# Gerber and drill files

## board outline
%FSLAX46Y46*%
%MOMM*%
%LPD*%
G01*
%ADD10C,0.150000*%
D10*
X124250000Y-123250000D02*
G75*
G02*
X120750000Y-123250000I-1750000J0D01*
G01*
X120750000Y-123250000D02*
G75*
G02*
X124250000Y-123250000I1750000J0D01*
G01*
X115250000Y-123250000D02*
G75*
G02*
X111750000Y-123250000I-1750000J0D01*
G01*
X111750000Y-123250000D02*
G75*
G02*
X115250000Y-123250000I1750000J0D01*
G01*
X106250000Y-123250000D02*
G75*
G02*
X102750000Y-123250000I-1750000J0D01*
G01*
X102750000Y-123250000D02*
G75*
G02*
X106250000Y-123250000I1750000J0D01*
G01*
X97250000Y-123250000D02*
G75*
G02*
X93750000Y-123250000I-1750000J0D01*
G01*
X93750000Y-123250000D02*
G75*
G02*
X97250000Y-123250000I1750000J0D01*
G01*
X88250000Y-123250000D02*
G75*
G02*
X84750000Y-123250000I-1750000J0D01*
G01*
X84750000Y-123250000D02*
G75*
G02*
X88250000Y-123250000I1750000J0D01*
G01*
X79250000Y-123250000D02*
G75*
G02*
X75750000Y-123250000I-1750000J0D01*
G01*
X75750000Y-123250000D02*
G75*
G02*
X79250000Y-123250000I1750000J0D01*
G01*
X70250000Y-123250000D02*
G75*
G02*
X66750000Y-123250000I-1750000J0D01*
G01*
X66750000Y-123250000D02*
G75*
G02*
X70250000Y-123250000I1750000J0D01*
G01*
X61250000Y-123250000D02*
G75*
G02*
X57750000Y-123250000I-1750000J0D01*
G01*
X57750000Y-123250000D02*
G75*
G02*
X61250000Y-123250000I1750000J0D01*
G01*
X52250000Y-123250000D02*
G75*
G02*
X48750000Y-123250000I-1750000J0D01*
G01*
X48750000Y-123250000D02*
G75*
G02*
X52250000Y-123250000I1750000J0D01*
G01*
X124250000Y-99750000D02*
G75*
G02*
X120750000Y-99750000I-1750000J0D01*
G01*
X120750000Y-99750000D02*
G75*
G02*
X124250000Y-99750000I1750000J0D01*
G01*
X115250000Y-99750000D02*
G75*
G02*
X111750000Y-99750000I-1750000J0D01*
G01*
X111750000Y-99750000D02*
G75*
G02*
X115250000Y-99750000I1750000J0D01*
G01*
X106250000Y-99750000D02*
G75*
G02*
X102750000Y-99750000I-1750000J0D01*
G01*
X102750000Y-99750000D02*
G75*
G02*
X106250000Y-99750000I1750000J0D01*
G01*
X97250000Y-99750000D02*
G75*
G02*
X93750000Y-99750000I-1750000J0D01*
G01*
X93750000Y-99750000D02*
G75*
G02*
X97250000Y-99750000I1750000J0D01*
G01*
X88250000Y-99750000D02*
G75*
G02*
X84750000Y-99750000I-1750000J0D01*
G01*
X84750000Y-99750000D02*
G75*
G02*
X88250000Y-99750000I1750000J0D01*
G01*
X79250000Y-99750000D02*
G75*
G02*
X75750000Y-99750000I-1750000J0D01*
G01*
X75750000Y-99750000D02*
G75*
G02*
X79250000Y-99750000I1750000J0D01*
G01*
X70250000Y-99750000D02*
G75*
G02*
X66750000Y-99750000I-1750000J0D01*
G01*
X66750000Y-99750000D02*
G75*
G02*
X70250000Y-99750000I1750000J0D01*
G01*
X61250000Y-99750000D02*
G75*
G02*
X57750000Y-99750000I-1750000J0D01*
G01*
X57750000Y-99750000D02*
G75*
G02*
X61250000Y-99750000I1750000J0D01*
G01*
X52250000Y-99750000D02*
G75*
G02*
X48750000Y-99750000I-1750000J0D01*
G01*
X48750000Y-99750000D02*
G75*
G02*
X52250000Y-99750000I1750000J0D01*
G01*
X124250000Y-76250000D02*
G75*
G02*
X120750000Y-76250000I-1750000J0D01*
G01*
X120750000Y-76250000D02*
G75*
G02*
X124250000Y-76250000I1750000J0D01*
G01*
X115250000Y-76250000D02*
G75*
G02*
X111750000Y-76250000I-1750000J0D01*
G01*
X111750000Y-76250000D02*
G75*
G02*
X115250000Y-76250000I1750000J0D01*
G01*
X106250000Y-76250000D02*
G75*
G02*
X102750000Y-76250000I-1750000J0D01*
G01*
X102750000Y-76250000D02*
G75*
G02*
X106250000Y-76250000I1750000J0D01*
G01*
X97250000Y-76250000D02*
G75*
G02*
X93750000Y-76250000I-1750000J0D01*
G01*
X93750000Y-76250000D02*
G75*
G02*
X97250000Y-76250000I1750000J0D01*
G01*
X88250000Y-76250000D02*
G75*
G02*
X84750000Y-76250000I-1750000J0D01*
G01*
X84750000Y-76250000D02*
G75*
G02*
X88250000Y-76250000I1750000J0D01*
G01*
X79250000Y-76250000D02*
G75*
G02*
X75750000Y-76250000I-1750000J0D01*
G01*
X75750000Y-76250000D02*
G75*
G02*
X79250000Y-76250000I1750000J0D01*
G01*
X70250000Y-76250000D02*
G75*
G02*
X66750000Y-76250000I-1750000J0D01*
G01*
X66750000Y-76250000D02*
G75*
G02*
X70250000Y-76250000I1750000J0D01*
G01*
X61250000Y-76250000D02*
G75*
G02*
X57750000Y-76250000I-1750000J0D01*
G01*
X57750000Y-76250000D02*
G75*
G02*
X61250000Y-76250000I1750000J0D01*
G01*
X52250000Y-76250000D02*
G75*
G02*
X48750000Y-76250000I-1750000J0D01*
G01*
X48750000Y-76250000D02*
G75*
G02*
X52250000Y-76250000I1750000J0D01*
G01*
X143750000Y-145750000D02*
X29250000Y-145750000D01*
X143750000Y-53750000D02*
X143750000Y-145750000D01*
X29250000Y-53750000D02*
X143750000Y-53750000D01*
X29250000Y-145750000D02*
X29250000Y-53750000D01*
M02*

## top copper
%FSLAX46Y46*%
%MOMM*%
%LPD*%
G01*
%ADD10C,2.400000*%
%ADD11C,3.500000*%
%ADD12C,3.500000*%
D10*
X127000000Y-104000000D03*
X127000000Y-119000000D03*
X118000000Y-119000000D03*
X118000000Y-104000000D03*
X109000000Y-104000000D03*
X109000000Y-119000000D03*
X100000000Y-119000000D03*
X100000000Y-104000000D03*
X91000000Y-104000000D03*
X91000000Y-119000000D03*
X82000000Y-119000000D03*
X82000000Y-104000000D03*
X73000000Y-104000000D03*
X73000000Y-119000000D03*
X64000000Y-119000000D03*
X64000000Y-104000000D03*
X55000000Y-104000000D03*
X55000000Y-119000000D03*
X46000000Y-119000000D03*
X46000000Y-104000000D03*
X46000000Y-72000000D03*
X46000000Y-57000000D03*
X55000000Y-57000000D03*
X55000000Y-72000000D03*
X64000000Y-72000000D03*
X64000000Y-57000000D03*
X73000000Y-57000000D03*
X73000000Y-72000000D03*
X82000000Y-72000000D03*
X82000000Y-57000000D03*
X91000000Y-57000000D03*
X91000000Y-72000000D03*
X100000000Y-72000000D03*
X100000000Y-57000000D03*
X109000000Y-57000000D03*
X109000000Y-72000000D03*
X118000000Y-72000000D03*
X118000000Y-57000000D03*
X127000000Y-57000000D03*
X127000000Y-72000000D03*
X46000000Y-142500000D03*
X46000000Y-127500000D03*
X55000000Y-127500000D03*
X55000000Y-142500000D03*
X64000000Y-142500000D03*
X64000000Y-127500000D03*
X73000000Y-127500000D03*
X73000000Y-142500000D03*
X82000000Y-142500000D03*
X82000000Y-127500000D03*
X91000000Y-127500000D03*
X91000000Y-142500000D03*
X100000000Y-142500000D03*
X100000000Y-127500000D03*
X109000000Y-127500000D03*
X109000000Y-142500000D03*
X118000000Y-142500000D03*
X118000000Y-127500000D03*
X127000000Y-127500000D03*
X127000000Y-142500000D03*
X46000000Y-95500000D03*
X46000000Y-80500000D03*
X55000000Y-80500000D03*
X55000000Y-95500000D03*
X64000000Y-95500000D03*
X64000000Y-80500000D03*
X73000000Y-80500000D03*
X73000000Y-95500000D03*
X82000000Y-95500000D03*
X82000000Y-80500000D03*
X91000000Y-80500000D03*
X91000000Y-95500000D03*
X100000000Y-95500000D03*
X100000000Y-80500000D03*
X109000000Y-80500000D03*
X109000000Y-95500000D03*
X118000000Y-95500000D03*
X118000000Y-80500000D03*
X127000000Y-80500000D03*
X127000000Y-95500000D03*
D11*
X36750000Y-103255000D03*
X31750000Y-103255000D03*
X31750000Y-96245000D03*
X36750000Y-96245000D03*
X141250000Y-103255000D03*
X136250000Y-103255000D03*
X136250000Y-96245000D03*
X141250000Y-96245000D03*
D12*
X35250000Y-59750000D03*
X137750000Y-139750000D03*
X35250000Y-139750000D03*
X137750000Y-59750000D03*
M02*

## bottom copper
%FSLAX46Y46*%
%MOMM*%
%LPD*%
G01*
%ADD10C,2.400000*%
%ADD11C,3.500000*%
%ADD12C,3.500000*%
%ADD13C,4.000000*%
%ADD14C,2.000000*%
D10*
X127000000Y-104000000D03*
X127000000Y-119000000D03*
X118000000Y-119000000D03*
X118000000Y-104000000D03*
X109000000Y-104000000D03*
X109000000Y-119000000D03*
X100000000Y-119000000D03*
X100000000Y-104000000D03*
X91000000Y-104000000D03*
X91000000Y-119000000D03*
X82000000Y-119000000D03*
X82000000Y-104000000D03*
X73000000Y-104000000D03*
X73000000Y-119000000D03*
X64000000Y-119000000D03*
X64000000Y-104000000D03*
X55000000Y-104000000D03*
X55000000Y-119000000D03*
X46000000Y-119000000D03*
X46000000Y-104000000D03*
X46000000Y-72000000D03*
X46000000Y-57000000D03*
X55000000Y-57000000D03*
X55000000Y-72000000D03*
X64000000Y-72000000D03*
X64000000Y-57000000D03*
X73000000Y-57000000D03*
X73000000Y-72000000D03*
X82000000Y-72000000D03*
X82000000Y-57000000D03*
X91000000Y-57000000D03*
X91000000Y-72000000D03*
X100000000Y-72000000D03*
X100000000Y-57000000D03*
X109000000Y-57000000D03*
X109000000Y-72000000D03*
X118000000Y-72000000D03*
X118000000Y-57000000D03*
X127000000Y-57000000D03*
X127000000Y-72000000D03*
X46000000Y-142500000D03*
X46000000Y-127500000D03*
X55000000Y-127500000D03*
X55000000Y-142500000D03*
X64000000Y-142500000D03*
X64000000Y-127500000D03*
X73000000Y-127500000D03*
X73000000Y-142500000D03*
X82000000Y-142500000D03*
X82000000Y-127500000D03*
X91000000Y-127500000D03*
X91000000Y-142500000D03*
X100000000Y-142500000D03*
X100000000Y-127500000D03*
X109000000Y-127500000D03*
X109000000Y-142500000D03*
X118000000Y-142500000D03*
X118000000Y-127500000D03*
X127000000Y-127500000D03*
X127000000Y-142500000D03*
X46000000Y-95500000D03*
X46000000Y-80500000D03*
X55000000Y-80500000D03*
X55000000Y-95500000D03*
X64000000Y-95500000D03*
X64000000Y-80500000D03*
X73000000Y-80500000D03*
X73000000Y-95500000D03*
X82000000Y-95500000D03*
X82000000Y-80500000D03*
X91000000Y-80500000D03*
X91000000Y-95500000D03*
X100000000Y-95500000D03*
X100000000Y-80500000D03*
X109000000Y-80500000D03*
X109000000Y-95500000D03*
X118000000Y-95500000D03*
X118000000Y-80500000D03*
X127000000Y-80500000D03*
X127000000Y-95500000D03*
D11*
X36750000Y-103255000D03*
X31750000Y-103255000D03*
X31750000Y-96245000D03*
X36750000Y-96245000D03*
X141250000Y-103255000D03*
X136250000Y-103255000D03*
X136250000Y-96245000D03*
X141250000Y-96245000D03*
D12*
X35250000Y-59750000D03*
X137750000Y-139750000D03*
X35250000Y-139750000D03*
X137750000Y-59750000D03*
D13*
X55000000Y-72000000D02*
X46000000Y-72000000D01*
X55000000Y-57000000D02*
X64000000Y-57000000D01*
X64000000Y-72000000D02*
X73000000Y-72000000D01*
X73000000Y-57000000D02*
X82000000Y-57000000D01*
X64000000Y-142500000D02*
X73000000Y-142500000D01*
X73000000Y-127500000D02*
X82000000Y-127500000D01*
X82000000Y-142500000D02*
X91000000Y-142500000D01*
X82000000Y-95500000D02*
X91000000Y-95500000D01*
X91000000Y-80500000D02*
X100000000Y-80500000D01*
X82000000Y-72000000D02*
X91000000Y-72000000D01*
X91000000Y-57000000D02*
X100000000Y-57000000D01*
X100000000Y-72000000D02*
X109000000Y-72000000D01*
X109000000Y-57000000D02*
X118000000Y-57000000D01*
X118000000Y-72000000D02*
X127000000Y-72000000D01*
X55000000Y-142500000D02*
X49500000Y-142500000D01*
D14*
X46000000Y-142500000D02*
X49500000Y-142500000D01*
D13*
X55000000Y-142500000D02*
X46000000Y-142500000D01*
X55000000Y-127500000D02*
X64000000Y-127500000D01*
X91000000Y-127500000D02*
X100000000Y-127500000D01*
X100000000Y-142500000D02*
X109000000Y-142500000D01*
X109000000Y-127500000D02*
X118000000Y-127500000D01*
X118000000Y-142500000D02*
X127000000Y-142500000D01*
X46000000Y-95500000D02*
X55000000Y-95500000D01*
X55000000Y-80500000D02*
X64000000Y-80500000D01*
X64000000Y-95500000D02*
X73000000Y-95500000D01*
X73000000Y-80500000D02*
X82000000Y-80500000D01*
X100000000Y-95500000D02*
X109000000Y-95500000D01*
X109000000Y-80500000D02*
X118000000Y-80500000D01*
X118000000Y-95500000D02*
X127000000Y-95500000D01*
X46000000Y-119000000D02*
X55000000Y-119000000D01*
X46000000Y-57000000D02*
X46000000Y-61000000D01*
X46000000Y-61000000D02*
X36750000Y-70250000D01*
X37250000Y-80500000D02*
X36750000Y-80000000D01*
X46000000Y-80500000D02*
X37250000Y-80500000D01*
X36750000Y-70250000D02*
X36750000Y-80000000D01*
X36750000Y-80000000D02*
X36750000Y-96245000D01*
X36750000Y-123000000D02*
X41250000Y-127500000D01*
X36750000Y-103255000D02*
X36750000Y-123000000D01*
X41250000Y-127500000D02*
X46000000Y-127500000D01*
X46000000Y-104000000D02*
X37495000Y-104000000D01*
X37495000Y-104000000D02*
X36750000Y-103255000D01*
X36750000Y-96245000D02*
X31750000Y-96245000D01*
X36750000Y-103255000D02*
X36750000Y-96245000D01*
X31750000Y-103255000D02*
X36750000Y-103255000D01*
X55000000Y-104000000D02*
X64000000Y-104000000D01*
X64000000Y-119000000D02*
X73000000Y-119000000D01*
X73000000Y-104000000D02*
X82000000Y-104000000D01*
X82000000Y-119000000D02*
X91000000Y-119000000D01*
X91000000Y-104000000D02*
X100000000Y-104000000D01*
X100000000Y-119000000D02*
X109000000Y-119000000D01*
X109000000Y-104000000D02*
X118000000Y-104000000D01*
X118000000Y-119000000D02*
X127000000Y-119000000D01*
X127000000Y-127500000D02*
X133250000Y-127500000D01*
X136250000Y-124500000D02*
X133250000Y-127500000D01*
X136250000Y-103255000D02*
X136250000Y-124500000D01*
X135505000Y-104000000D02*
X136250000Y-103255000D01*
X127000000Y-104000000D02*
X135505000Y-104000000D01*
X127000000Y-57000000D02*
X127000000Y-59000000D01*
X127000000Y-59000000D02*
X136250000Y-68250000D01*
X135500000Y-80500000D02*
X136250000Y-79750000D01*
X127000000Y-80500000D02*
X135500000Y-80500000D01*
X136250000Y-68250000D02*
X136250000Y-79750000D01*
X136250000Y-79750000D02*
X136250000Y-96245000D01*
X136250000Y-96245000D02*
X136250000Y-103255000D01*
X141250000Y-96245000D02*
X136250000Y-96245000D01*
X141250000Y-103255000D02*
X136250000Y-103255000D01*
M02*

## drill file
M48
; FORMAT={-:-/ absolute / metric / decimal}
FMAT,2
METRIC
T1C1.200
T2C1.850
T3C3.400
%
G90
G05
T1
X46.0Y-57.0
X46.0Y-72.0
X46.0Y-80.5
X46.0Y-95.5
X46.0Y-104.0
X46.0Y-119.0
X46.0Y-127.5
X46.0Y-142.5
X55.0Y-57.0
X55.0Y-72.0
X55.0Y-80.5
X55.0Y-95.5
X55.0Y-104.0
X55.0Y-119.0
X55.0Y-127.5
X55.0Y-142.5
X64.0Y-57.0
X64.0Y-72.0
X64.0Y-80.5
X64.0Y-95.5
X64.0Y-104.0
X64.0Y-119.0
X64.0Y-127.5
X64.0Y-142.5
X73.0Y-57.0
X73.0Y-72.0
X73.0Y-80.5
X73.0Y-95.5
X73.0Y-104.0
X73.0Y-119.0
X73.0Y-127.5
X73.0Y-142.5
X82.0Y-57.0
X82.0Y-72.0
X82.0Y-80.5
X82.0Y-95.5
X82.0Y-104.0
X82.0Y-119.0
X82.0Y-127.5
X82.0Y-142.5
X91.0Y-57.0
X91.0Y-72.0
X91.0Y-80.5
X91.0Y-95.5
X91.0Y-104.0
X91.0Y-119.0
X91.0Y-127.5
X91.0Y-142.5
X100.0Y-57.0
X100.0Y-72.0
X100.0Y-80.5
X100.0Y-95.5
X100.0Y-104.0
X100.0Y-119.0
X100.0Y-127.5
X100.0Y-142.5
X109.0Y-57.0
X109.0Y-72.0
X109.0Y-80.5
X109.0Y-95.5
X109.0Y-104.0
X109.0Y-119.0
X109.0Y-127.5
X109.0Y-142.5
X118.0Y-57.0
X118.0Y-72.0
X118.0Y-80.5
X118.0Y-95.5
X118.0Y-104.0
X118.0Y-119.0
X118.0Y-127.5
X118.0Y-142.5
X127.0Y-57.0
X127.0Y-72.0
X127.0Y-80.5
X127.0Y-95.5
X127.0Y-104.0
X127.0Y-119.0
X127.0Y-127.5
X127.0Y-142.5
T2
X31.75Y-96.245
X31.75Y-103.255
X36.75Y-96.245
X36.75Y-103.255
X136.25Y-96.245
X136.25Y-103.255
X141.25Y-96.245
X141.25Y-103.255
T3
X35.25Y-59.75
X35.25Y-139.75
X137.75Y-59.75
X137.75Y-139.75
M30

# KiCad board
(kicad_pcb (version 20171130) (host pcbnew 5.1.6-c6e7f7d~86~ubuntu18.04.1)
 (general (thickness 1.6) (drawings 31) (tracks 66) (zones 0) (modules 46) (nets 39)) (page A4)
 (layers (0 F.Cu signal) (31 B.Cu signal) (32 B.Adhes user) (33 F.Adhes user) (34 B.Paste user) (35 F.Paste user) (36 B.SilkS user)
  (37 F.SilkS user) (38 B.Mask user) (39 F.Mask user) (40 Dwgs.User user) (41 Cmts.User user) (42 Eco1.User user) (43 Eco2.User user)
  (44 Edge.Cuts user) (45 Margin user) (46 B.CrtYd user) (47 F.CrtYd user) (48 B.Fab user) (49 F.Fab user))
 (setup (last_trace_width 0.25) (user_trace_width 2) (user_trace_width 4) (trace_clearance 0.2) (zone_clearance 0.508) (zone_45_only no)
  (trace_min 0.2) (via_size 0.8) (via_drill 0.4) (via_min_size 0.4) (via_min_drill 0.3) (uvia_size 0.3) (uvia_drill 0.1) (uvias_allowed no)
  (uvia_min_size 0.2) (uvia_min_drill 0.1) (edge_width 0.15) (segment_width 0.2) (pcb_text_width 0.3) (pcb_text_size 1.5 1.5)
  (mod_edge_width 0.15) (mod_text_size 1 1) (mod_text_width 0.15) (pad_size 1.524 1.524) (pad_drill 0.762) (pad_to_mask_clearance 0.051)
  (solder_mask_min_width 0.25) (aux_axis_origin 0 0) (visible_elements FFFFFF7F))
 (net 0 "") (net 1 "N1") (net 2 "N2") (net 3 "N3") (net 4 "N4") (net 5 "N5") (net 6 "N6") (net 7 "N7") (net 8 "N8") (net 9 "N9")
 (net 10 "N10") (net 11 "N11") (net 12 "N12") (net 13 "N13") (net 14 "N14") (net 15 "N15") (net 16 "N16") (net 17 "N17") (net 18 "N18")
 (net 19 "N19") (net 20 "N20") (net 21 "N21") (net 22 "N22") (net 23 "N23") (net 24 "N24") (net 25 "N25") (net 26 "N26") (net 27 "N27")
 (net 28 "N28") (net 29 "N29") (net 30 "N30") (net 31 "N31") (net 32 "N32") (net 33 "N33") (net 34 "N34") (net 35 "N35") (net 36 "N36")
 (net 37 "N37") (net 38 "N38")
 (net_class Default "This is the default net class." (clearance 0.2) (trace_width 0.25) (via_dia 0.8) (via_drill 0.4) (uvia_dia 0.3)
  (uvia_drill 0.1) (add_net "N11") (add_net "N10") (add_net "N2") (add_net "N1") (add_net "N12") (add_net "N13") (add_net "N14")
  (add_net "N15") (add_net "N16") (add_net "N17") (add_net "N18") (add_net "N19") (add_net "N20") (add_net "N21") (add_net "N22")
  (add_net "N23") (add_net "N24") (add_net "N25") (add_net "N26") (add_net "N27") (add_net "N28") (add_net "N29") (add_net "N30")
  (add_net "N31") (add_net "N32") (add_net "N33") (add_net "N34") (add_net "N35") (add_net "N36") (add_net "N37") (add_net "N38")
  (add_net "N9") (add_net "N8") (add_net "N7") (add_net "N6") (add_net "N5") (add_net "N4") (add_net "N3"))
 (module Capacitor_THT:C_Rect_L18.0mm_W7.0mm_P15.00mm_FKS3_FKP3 (layer F.Cu) (at 127 119 90)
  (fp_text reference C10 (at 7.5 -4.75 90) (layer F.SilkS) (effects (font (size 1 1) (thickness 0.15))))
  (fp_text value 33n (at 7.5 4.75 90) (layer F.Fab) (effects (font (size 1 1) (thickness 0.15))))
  (pad 2 thru_hole circle (at 15 0 90) (size 2.4 2.4) (drill 1.2) (layers *.Cu *.Mask) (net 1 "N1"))
  (pad 1 thru_hole circle (at 0 0 90) (size 2.4 2.4) (drill 1.2) (layers *.Cu *.Mask) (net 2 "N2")))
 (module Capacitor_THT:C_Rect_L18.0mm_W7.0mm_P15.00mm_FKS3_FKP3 (layer F.Cu) (at 118 104 270)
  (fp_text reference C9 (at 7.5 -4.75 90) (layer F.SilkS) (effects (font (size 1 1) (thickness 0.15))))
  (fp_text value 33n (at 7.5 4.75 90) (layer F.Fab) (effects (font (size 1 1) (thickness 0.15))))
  (pad 2 thru_hole circle (at 15 0 270) (size 2.4 2.4) (drill 1.2) (layers *.Cu *.Mask) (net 2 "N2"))
  (pad 1 thru_hole circle (at 0 0 270) (size 2.4 2.4) (drill 1.2) (layers *.Cu *.Mask) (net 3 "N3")))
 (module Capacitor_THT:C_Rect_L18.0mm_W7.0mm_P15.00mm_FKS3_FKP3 (layer F.Cu) (at 109 119 90)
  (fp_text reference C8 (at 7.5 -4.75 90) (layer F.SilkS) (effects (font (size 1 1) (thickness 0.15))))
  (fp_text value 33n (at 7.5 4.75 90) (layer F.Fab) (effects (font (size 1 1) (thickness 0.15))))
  (pad 2 thru_hole circle (at 15 0 90) (size 2.4 2.4) (drill 1.2) (layers *.Cu *.Mask) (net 3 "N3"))
  (pad 1 thru_hole circle (at 0 0 90) (size 2.4 2.4) (drill 1.2) (layers *.Cu *.Mask) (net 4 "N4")))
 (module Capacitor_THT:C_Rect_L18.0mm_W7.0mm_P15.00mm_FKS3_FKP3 (layer F.Cu) (at 100 104 270)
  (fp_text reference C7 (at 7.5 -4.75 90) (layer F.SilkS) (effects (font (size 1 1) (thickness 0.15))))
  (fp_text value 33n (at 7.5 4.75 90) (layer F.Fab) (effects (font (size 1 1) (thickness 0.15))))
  (pad 2 thru_hole circle (at 15 0 270) (size 2.4 2.4) (drill 1.2) (layers *.Cu *.Mask) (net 4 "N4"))
  (pad 1 thru_hole circle (at 0 0 270) (size 2.4 2.4) (drill 1.2) (layers *.Cu *.Mask) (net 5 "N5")))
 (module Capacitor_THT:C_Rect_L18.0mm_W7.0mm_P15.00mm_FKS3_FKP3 (layer F.Cu) (at 91 119 90)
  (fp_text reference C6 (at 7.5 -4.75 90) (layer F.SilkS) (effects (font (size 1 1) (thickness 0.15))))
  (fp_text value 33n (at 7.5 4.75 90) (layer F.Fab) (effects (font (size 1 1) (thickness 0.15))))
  (pad 2 thru_hole circle (at 15 0 90) (size 2.4 2.4) (drill 1.2) (layers *.Cu *.Mask) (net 5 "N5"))
  (pad 1 thru_hole circle (at 0 0 90) (size 2.4 2.4) (drill 1.2) (layers *.Cu *.Mask) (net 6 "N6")))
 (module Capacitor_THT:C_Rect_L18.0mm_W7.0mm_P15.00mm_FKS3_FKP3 (layer F.Cu) (at 82 104 270)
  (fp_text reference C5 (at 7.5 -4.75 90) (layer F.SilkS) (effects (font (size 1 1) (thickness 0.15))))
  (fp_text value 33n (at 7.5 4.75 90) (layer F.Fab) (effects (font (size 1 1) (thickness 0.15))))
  (pad 2 thru_hole circle (at 15 0 270) (size 2.4 2.4) (drill 1.2) (layers *.Cu *.Mask) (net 6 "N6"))
  (pad 1 thru_hole circle (at 0 0 270) (size 2.4 2.4) (drill 1.2) (layers *.Cu *.Mask) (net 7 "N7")))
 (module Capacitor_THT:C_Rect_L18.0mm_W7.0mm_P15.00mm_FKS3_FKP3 (layer F.Cu) (at 73 119 90)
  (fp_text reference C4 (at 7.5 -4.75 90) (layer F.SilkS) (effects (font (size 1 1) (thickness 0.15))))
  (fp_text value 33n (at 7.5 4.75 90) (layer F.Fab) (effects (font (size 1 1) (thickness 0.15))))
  (pad 2 thru_hole circle (at 15 0 90) (size 2.4 2.4) (drill 1.2) (layers *.Cu *.Mask) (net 7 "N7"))
  (pad 1 thru_hole circle (at 0 0 90) (size 2.4 2.4) (drill 1.2) (layers *.Cu *.Mask) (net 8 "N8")))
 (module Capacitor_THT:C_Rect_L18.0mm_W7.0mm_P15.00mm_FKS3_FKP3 (layer F.Cu) (at 64 104 270)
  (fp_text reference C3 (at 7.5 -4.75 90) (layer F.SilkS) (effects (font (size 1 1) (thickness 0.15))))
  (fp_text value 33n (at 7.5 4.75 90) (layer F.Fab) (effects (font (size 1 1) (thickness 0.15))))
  (pad 2 thru_hole circle (at 15 0 270) (size 2.4 2.4) (drill 1.2) (layers *.Cu *.Mask) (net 8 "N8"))
  (pad 1 thru_hole circle (at 0 0 270) (size 2.4 2.4) (drill 1.2) (layers *.Cu *.Mask) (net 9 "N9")))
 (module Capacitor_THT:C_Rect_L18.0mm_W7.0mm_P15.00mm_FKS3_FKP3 (layer F.Cu) (at 55 119 90)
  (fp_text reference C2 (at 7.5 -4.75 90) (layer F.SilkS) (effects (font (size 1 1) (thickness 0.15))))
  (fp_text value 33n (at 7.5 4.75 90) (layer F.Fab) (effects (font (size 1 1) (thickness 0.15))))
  (pad 2 thru_hole circle (at 15 0 90) (size 2.4 2.4) (drill 1.2) (layers *.Cu *.Mask) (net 9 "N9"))
  (pad 1 thru_hole circle (at 0 0 90) (size 2.4 2.4) (drill 1.2) (layers *.Cu *.Mask) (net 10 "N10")))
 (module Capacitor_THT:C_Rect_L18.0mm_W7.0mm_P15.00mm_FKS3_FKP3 (layer F.Cu) (at 46 104 270)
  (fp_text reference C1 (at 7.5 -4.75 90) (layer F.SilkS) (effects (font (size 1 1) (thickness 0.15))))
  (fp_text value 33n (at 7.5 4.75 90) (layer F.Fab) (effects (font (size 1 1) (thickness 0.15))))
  (pad 2 thru_hole circle (at 15 0 270) (size 2.4 2.4) (drill 1.2) (layers *.Cu *.Mask) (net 10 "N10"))
  (pad 1 thru_hole circle (at 0 0 270) (size 2.4 2.4) (drill 1.2) (layers *.Cu *.Mask) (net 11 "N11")))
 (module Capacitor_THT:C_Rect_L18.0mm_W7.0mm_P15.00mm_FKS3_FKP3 (layer F.Cu) (at 46 57 270)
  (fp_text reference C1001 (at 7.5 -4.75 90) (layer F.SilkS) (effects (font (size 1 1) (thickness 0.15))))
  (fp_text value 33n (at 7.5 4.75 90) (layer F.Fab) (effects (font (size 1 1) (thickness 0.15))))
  (pad 2 thru_hole circle (at 15 0 270) (size 2.4 2.4) (drill 1.2) (layers *.Cu *.Mask) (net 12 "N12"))
  (pad 1 thru_hole circle (at 0 0 270) (size 2.4 2.4) (drill 1.2) (layers *.Cu *.Mask) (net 11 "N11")))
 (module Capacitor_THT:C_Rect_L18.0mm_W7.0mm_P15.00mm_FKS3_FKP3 (layer F.Cu) (at 55 72 90)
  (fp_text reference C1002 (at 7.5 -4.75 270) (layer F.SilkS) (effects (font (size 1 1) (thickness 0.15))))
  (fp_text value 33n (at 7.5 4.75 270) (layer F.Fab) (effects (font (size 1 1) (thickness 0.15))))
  (pad 2 thru_hole circle (at 15 0 90) (size 2.4 2.4) (drill 1.2) (layers *.Cu *.Mask) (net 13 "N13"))
  (pad 1 thru_hole circle (at 0 0 90) (size 2.4 2.4) (drill 1.2) (layers *.Cu *.Mask) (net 12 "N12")))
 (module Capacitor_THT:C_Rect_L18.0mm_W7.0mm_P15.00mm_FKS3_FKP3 (layer F.Cu) (at 64 57 270)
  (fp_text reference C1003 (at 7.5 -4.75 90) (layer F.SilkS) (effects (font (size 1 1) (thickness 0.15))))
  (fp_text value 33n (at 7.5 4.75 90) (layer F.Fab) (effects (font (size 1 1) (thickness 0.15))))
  (pad 2 thru_hole circle (at 15 0 270) (size 2.4 2.4) (drill 1.2) (layers *.Cu *.Mask) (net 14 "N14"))
  (pad 1 thru_hole circle (at 0 0 270) (size 2.4 2.4) (drill 1.2) (layers *.Cu *.Mask) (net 13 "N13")))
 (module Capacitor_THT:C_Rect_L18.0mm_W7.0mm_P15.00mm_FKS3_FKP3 (layer F.Cu) (at 73 72 90)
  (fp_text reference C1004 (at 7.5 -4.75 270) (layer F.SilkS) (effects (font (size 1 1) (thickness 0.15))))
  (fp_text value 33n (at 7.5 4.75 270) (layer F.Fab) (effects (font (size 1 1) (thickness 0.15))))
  (pad 2 thru_hole circle (at 15 0 90) (size 2.4 2.4) (drill 1.2) (layers *.Cu *.Mask) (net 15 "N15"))
  (pad 1 thru_hole circle (at 0 0 90) (size 2.4 2.4) (drill 1.2) (layers *.Cu *.Mask) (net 14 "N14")))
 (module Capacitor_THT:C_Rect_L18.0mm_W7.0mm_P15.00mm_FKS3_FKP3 (layer F.Cu) (at 82 57 270)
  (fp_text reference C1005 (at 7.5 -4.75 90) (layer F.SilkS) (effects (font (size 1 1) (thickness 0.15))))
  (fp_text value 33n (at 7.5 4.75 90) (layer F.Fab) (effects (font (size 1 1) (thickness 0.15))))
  (pad 2 thru_hole circle (at 15 0 270) (size 2.4 2.4) (drill 1.2) (layers *.Cu *.Mask) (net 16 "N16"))
  (pad 1 thru_hole circle (at 0 0 270) (size 2.4 2.4) (drill 1.2) (layers *.Cu *.Mask) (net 15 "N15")))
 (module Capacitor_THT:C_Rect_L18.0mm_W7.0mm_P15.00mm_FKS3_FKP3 (layer F.Cu) (at 91 72 90)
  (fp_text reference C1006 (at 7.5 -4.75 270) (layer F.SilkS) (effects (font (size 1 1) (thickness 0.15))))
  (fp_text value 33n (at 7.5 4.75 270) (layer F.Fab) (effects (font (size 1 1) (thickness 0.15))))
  (pad 2 thru_hole circle (at 15 0 90) (size 2.4 2.4) (drill 1.2) (layers *.Cu *.Mask) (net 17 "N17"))
  (pad 1 thru_hole circle (at 0 0 90) (size 2.4 2.4) (drill 1.2) (layers *.Cu *.Mask) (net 16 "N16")))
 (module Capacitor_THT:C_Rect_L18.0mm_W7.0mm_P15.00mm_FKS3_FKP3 (layer F.Cu) (at 100 57 270)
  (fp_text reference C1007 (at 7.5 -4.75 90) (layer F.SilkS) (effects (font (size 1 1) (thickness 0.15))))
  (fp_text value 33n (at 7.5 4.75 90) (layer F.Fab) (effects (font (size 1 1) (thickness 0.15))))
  (pad 2 thru_hole circle (at 15 0 270) (size 2.4 2.4) (drill 1.2) (layers *.Cu *.Mask) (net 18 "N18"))
  (pad 1 thru_hole circle (at 0 0 270) (size 2.4 2.4) (drill 1.2) (layers *.Cu *.Mask) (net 17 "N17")))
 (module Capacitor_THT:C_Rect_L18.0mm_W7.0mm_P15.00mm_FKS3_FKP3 (layer F.Cu) (at 109 72 90)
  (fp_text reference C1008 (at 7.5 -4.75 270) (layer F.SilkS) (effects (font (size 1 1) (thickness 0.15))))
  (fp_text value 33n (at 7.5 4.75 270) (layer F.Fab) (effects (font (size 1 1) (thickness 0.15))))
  (pad 2 thru_hole circle (at 15 0 90) (size 2.4 2.4) (drill 1.2) (layers *.Cu *.Mask) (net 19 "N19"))
  (pad 1 thru_hole circle (at 0 0 90) (size 2.4 2.4) (drill 1.2) (layers *.Cu *.Mask) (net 18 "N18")))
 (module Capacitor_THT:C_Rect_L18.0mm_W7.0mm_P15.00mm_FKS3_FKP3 (layer F.Cu) (at 118 57 270)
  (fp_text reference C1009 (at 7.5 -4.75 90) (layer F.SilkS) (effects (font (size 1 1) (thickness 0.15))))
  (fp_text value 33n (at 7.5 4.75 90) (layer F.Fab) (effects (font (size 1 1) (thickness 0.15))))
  (pad 2 thru_hole circle (at 15 0 270) (size 2.4 2.4) (drill 1.2) (layers *.Cu *.Mask) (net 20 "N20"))
  (pad 1 thru_hole circle (at 0 0 270) (size 2.4 2.4) (drill 1.2) (layers *.Cu *.Mask) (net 19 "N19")))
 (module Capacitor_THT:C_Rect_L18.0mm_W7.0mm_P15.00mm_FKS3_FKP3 (layer F.Cu) (at 127 72 90)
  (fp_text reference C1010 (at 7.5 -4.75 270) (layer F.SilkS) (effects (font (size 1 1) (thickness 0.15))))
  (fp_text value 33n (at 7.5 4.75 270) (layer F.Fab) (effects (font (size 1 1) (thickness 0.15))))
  (pad 2 thru_hole circle (at 15 0 90) (size 2.4 2.4) (drill 1.2) (layers *.Cu *.Mask) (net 1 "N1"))
  (pad 1 thru_hole circle (at 0 0 90) (size 2.4 2.4) (drill 1.2) (layers *.Cu *.Mask) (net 20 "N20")))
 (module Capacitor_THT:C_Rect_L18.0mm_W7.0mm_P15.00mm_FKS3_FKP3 (layer F.Cu) (at 46 127.5 270)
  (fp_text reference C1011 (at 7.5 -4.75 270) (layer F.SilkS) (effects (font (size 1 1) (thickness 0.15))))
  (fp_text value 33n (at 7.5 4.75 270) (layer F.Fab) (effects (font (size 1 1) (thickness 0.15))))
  (pad 2 thru_hole circle (at 15 0 270) (size 2.4 2.4) (drill 1.2) (layers *.Cu *.Mask) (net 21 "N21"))
  (pad 1 thru_hole circle (at 0 0 270) (size 2.4 2.4) (drill 1.2) (layers *.Cu *.Mask) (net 11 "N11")))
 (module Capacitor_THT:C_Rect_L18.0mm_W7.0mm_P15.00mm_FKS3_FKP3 (layer F.Cu) (at 55 142.5 90)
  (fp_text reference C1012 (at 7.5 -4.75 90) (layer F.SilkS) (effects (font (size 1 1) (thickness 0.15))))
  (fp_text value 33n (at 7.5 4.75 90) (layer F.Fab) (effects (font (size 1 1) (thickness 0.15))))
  (pad 2 thru_hole circle (at 15 0 90) (size 2.4 2.4) (drill 1.2) (layers *.Cu *.Mask) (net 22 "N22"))
  (pad 1 thru_hole circle (at 0 0 90) (size 2.4 2.4) (drill 1.2) (layers *.Cu *.Mask) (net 21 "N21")))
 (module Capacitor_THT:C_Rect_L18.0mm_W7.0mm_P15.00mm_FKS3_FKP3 (layer F.Cu) (at 64 127.5 270)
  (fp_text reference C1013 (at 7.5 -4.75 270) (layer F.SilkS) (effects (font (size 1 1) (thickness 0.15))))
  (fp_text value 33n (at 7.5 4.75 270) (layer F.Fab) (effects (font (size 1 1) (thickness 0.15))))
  (pad 2 thru_hole circle (at 15 0 270) (size 2.4 2.4) (drill 1.2) (layers *.Cu *.Mask) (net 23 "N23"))
  (pad 1 thru_hole circle (at 0 0 270) (size 2.4 2.4) (drill 1.2) (layers *.Cu *.Mask) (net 22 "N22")))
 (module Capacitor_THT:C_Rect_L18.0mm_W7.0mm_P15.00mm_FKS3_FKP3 (layer F.Cu) (at 73 142.5 90)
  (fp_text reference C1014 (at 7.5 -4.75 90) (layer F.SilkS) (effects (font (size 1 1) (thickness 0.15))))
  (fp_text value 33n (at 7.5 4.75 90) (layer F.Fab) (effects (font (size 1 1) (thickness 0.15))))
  (pad 2 thru_hole circle (at 15 0 90) (size 2.4 2.4) (drill 1.2) (layers *.Cu *.Mask) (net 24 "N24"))
  (pad 1 thru_hole circle (at 0 0 90) (size 2.4 2.4) (drill 1.2) (layers *.Cu *.Mask) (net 23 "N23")))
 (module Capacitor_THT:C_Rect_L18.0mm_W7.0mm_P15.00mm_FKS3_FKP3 (layer F.Cu) (at 82 127.5 270)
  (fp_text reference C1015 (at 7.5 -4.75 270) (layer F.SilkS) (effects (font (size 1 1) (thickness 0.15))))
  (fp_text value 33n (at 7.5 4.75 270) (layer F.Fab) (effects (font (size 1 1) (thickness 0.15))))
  (pad 2 thru_hole circle (at 15 0 270) (size 2.4 2.4) (drill 1.2) (layers *.Cu *.Mask) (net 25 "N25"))
  (pad 1 thru_hole circle (at 0 0 270) (size 2.4 2.4) (drill 1.2) (layers *.Cu *.Mask) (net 24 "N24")))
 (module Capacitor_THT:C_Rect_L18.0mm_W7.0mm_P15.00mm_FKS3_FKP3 (layer F.Cu) (at 91 142.5 90)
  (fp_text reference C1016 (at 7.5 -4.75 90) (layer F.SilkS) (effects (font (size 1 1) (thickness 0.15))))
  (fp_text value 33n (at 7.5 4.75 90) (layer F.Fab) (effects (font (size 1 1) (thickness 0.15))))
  (pad 2 thru_hole circle (at 15 0 90) (size 2.4 2.4) (drill 1.2) (layers *.Cu *.Mask) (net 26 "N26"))
  (pad 1 thru_hole circle (at 0 0 90) (size 2.4 2.4) (drill 1.2) (layers *.Cu *.Mask) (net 25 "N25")))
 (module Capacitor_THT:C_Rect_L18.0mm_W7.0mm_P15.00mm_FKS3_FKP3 (layer F.Cu) (at 100 127.5 270)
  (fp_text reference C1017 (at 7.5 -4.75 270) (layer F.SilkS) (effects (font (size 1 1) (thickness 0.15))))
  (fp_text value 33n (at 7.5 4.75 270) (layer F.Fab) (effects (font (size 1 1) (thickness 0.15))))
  (pad 2 thru_hole circle (at 15 0 270) (size 2.4 2.4) (drill 1.2) (layers *.Cu *.Mask) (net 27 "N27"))
  (pad 1 thru_hole circle (at 0 0 270) (size 2.4 2.4) (drill 1.2) (layers *.Cu *.Mask) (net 26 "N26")))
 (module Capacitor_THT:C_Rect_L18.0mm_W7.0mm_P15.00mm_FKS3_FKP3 (layer F.Cu) (at 109 142.5 90)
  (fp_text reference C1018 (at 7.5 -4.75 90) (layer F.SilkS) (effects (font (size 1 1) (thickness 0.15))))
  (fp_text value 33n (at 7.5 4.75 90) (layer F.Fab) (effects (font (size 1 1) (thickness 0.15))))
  (pad 2 thru_hole circle (at 15 0 90) (size 2.4 2.4) (drill 1.2) (layers *.Cu *.Mask) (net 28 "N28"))
  (pad 1 thru_hole circle (at 0 0 90) (size 2.4 2.4) (drill 1.2) (layers *.Cu *.Mask) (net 27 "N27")))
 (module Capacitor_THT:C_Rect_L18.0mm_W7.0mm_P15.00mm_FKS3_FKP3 (layer F.Cu) (at 118 127.5 270)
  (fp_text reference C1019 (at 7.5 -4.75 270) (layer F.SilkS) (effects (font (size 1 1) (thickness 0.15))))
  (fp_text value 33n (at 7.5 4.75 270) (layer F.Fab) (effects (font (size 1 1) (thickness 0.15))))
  (pad 2 thru_hole circle (at 15 0 270) (size 2.4 2.4) (drill 1.2) (layers *.Cu *.Mask) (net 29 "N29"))
  (pad 1 thru_hole circle (at 0 0 270) (size 2.4 2.4) (drill 1.2) (layers *.Cu *.Mask) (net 28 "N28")))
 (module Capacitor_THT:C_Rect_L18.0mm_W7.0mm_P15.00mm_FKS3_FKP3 (layer F.Cu) (at 127 142.5 90)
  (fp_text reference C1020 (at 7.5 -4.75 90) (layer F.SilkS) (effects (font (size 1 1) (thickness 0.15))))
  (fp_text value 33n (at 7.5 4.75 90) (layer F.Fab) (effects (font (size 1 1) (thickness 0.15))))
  (pad 2 thru_hole circle (at 15 0 90) (size 2.4 2.4) (drill 1.2) (layers *.Cu *.Mask) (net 1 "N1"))
  (pad 1 thru_hole circle (at 0 0 90) (size 2.4 2.4) (drill 1.2) (layers *.Cu *.Mask) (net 29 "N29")))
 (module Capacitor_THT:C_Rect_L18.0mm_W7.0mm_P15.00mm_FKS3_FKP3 (layer F.Cu) (at 46 80.5 270)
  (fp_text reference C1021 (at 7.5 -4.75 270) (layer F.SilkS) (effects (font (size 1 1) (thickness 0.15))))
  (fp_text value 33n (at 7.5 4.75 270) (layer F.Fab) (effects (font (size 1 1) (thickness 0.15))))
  (pad 2 thru_hole circle (at 15 0 270) (size 2.4 2.4) (drill 1.2) (layers *.Cu *.Mask) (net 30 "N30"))
  (pad 1 thru_hole circle (at 0 0 270) (size 2.4 2.4) (drill 1.2) (layers *.Cu *.Mask) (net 11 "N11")))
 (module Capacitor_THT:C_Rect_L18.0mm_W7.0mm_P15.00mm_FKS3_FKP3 (layer F.Cu) (at 55 95.5 90)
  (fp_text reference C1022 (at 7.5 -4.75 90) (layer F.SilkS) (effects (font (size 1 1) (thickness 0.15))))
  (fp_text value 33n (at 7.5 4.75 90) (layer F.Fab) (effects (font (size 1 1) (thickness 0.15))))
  (pad 2 thru_hole circle (at 15 0 90) (size 2.4 2.4) (drill 1.2) (layers *.Cu *.Mask) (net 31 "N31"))
  (pad 1 thru_hole circle (at 0 0 90) (size 2.4 2.4) (drill 1.2) (layers *.Cu *.Mask) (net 30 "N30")))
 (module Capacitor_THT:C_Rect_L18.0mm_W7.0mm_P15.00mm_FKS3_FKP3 (layer F.Cu) (at 64 80.5 270)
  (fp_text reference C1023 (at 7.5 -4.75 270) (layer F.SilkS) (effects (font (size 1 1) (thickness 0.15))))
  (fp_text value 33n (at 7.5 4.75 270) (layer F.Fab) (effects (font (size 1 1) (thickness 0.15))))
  (pad 2 thru_hole circle (at 15 0 270) (size 2.4 2.4) (drill 1.2) (layers *.Cu *.Mask) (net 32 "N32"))
  (pad 1 thru_hole circle (at 0 0 270) (size 2.4 2.4) (drill 1.2) (layers *.Cu *.Mask) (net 31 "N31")))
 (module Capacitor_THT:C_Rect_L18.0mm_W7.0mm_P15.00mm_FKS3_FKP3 (layer F.Cu) (at 73 95.5 90)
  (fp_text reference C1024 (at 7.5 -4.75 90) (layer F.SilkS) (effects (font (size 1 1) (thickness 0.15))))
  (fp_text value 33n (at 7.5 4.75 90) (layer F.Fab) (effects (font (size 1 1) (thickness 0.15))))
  (pad 2 thru_hole circle (at 15 0 90) (size 2.4 2.4) (drill 1.2) (layers *.Cu *.Mask) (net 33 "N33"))
  (pad 1 thru_hole circle (at 0 0 90) (size 2.4 2.4) (drill 1.2) (layers *.Cu *.Mask) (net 32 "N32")))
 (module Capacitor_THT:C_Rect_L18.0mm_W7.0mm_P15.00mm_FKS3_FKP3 (layer F.Cu) (at 82 80.5 270)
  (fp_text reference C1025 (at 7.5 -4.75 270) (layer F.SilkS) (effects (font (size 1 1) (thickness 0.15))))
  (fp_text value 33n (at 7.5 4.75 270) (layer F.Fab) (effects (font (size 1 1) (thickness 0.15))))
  (pad 2 thru_hole circle (at 15 0 270) (size 2.4 2.4) (drill 1.2) (layers *.Cu *.Mask) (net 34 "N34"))
  (pad 1 thru_hole circle (at 0 0 270) (size 2.4 2.4) (drill 1.2) (layers *.Cu *.Mask) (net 33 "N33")))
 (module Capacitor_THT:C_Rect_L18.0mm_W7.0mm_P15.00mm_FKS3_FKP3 (layer F.Cu) (at 91 95.5 90)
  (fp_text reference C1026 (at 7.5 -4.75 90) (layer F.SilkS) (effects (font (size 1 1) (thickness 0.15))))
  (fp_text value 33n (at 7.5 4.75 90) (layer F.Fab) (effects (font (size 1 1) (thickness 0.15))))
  (pad 2 thru_hole circle (at 15 0 90) (size 2.4 2.4) (drill 1.2) (layers *.Cu *.Mask) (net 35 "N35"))
  (pad 1 thru_hole circle (at 0 0 90) (size 2.4 2.4) (drill 1.2) (layers *.Cu *.Mask) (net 34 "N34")))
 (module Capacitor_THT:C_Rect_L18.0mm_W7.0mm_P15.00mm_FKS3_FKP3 (layer F.Cu) (at 100 80.5 270)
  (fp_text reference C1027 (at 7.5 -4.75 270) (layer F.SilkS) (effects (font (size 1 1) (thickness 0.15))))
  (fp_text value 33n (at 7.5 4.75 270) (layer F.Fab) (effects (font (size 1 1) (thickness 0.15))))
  (pad 2 thru_hole circle (at 15 0 270) (size 2.4 2.4) (drill 1.2) (layers *.Cu *.Mask) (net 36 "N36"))
  (pad 1 thru_hole circle (at 0 0 270) (size 2.4 2.4) (drill 1.2) (layers *.Cu *.Mask) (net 35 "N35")))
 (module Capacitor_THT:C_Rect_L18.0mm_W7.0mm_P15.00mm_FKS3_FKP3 (layer F.Cu) (at 109 95.5 90)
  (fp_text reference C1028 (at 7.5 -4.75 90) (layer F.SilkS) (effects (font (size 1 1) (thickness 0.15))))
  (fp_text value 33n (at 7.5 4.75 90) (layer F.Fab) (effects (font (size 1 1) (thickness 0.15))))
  (pad 2 thru_hole circle (at 15 0 90) (size 2.4 2.4) (drill 1.2) (layers *.Cu *.Mask) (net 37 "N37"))
  (pad 1 thru_hole circle (at 0 0 90) (size 2.4 2.4) (drill 1.2) (layers *.Cu *.Mask) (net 36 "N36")))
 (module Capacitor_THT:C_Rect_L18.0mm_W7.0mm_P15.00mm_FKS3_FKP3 (layer F.Cu) (at 118 80.5 270)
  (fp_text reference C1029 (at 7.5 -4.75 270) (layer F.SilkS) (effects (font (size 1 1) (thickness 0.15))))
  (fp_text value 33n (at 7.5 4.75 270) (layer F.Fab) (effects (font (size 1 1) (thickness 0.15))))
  (pad 2 thru_hole circle (at 15 0 270) (size 2.4 2.4) (drill 1.2) (layers *.Cu *.Mask) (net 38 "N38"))
  (pad 1 thru_hole circle (at 0 0 270) (size 2.4 2.4) (drill 1.2) (layers *.Cu *.Mask) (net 37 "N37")))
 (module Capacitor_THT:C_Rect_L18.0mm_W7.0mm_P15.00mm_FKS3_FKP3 (layer F.Cu) (at 127 95.5 90)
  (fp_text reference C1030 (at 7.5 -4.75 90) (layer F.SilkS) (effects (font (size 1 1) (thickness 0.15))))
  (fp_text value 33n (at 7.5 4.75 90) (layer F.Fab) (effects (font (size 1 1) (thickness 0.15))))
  (pad 2 thru_hole circle (at 15 0 90) (size 2.4 2.4) (drill 1.2) (layers *.Cu *.Mask) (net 1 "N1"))
  (pad 1 thru_hole circle (at 0 0 90) (size 2.4 2.4) (drill 1.2) (layers *.Cu *.Mask) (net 38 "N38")))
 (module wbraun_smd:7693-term (layer F.Cu) (at 34.25 99.75)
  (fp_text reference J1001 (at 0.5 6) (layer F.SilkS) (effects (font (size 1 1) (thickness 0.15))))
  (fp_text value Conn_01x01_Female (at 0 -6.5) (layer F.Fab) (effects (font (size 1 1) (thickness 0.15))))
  (pad 1 thru_hole circle (at 2.5 3.505) (size 3.5 3.5) (drill 1.85) (layers *.Cu *.Mask) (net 11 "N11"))
  (pad 1 thru_hole circle (at -2.5 3.505) (size 3.5 3.5) (drill 1.85) (layers *.Cu *.Mask) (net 11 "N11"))
  (pad 1 thru_hole circle (at -2.5 -3.505) (size 3.5 3.5) (drill 1.85) (layers *.Cu *.Mask) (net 11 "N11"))
  (pad 1 thru_hole circle (at 2.5 -3.505) (size 3.5 3.5) (drill 1.85) (layers *.Cu *.Mask) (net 11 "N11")))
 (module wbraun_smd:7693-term (layer F.Cu) (at 138.75 99.75)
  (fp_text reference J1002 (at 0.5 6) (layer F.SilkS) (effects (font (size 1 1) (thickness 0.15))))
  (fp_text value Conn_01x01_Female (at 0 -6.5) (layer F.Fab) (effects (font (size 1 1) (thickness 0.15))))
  (pad 1 thru_hole circle (at 2.5 3.505) (size 3.5 3.5) (drill 1.85) (layers *.Cu *.Mask) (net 1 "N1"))
  (pad 1 thru_hole circle (at -2.5 3.505) (size 3.5 3.5) (drill 1.85) (layers *.Cu *.Mask) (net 1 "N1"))
  (pad 1 thru_hole circle (at -2.5 -3.505) (size 3.5 3.5) (drill 1.85) (layers *.Cu *.Mask) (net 1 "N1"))
  (pad 1 thru_hole circle (at 2.5 -3.505) (size 3.5 3.5) (drill 1.85) (layers *.Cu *.Mask) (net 1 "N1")))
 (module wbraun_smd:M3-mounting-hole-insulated (layer F.Cu) (at 35.25 59.75)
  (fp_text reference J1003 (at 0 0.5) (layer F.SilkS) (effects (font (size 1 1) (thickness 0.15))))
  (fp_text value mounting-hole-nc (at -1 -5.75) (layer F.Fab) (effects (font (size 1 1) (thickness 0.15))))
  (pad "" np_thru_hole circle (at 0 0) (size 3.5 3.5) (drill 3.4) (layers *.Cu *.Mask)))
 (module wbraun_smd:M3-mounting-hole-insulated (layer F.Cu) (at 137.75 139.75)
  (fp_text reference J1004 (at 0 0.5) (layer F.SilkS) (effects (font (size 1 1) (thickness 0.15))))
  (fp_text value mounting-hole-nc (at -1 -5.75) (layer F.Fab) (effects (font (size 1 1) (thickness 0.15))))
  (pad "" np_thru_hole circle (at 0 0) (size 3.5 3.5) (drill 3.4) (layers *.Cu *.Mask)))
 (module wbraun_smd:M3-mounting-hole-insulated (layer F.Cu) (at 35.25 139.75)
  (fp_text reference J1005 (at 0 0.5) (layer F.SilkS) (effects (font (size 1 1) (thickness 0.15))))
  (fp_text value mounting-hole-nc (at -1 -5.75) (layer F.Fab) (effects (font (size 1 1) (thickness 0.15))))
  (pad "" np_thru_hole circle (at 0 0) (size 3.5 3.5) (drill 3.4) (layers *.Cu *.Mask)))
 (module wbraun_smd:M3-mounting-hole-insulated (layer F.Cu) (at 137.75 59.75)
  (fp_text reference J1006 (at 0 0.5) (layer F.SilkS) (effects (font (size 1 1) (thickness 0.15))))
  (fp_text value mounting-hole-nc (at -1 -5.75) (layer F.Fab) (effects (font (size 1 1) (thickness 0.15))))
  (pad "" np_thru_hole circle (at 0 0) (size 3.5 3.5) (drill 3.4) (layers *.Cu *.Mask)))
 (gr_circle (center 122.5 123.25) (end 122.5 125) (layer Edge.Cuts) (width 0.15))
 (gr_circle (center 113.5 123.25) (end 113.5 125) (layer Edge.Cuts) (width 0.15))
 (gr_circle (center 104.5 123.25) (end 104.5 125) (layer Edge.Cuts) (width 0.15))
 (gr_circle (center 95.5 123.25) (end 95.5 125) (layer Edge.Cuts) (width 0.15))
 (gr_circle (center 86.5 123.25) (end 86.5 125) (layer Edge.Cuts) (width 0.15))
 (gr_circle (center 77.5 123.25) (end 77.5 125) (layer Edge.Cuts) (width 0.15))
 (gr_circle (center 68.5 123.25) (end 68.5 125) (layer Edge.Cuts) (width 0.15))
 (gr_circle (center 59.5 123.25) (end 59.5 125) (layer Edge.Cuts) (width 0.15))
 (gr_circle (center 50.5 123.25) (end 50.5 125) (layer Edge.Cuts) (width 0.15))
 (gr_circle (center 122.5 99.75) (end 122.5 101.5) (layer Edge.Cuts) (width 0.15))
 (gr_circle (center 113.5 99.75) (end 113.5 101.5) (layer Edge.Cuts) (width 0.15))
 (gr_circle (center 104.5 99.75) (end 104.5 101.5) (layer Edge.Cuts) (width 0.15))
 (gr_circle (center 95.5 99.75) (end 95.5 101.5) (layer Edge.Cuts) (width 0.15))
 (gr_circle (center 86.5 99.75) (end 86.5 101.5) (layer Edge.Cuts) (width 0.15))
 (gr_circle (center 77.5 99.75) (end 77.5 101.5) (layer Edge.Cuts) (width 0.15))
 (gr_circle (center 68.5 99.75) (end 68.5 101.5) (layer Edge.Cuts) (width 0.15))
 (gr_circle (center 59.5 99.75) (end 59.5 101.5) (layer Edge.Cuts) (width 0.15))
 (gr_circle (center 50.5 99.75) (end 50.5 101.5) (layer Edge.Cuts) (width 0.15))
 (gr_circle (center 122.5 76.25) (end 122.5 78) (layer Edge.Cuts) (width 0.15))
 (gr_circle (center 113.5 76.25) (end 113.5 78) (layer Edge.Cuts) (width 0.15))
 (gr_circle (center 104.5 76.25) (end 104.5 78) (layer Edge.Cuts) (width 0.15))
 (gr_circle (center 95.5 76.25) (end 95.5 78) (layer Edge.Cuts) (width 0.15))
 (gr_circle (center 86.5 76.25) (end 86.5 78) (layer Edge.Cuts) (width 0.15))
 (gr_circle (center 77.5 76.25) (end 77.5 78) (layer Edge.Cuts) (width 0.15))
 (gr_circle (center 68.5 76.25) (end 68.5 78) (layer Edge.Cuts) (width 0.15))
 (gr_circle (center 59.5 76.25) (end 59.5 78) (layer Edge.Cuts) (width 0.15))
 (gr_circle (center 50.5 76.25) (end 50.5 78) (layer Edge.Cuts) (width 0.15))
 (gr_line (start 143.75 145.75) (end 29.25 145.75) (layer Edge.Cuts) (width 0.15))
 (gr_line (start 143.75 53.75) (end 143.75 145.75) (layer Edge.Cuts) (width 0.15))
 (gr_line (start 29.25 53.75) (end 143.75 53.75) (layer Edge.Cuts) (width 0.15))
 (gr_line (start 29.25 145.75) (end 29.25 53.75) (layer Edge.Cuts) (width 0.15))
 (segment (start 55 72) (end 46 72) (width 4) (layer B.Cu) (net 12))
 (segment (start 55 57) (end 64 57) (width 4) (layer B.Cu) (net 13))
 (segment (start 64 72) (end 73 72) (width 4) (layer B.Cu) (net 14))
 (segment (start 73 57) (end 82 57) (width 4) (layer B.Cu) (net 15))
 (segment (start 64 142.5) (end 73 142.5) (width 4) (layer B.Cu) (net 23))
 (segment (start 73 127.5) (end 82 127.5) (width 4) (layer B.Cu) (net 24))
 (segment (start 82 142.5) (end 91 142.5) (width 4) (layer B.Cu) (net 25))
 (segment (start 82 95.5) (end 91 95.5) (width 4) (layer B.Cu) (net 34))
 (segment (start 91 80.5) (end 100 80.5) (width 4) (layer B.Cu) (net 35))
 (segment (start 82 72) (end 91 72) (width 4) (layer B.Cu) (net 16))
 (segment (start 91 57) (end 100 57) (width 4) (layer B.Cu) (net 17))
 (segment (start 100 72) (end 109 72) (width 4) (layer B.Cu) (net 18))
 (segment (start 109 57) (end 118 57) (width 4) (layer B.Cu) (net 19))
 (segment (start 118 72) (end 127 72) (width 4) (layer B.Cu) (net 20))
 (segment (start 55 142.5) (end 49.5 142.5) (width 4) (layer B.Cu) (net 21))
 (segment (start 46 142.5) (end 49.5 142.5) (width 2) (layer B.Cu) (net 21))
 (segment (start 55 142.5) (end 46 142.5) (width 4) (layer B.Cu) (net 21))
 (segment (start 55 127.5) (end 64 127.5) (width 4) (layer B.Cu) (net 22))
 (segment (start 91 127.5) (end 100 127.5) (width 4) (layer B.Cu) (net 26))
 (segment (start 100 142.5) (end 109 142.5) (width 4) (layer B.Cu) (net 27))
 (segment (start 109 127.5) (end 118 127.5) (width 4) (layer B.Cu) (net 28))
 (segment (start 118 142.5) (end 127 142.5) (width 4) (layer B.Cu) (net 29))
 (segment (start 46 95.5) (end 55 95.5) (width 4) (layer B.Cu) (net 30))
 (segment (start 55 80.5) (end 64 80.5) (width 4) (layer B.Cu) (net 31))
 (segment (start 64 95.5) (end 73 95.5) (width 4) (layer B.Cu) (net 32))
 (segment (start 73 80.5) (end 82 80.5) (width 4) (layer B.Cu) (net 33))
 (segment (start 100 95.5) (end 109 95.5) (width 4) (layer B.Cu) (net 36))
 (segment (start 109 80.5) (end 118 80.5) (width 4) (layer B.Cu) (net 37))
 (segment (start 118 95.5) (end 127 95.5) (width 4) (layer B.Cu) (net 38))
 (segment (start 46 119) (end 55 119) (width 4) (layer B.Cu) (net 10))
 (segment (start 46 57) (end 46 61) (width 4) (layer B.Cu) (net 11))
 (segment (start 46 61) (end 36.75 70.25) (width 4) (layer B.Cu) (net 11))
 (segment (start 37.25 80.5) (end 36.75 80) (width 4) (layer B.Cu) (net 11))
 (segment (start 46 80.5) (end 37.25 80.5) (width 4) (layer B.Cu) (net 11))
 (segment (start 36.75 70.25) (end 36.75 80) (width 4) (layer B.Cu) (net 11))
 (segment (start 36.75 80) (end 36.75 96.245) (width 4) (layer B.Cu) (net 11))
 (segment (start 36.75 123) (end 41.25 127.5) (width 4) (layer B.Cu) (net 11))
 (segment (start 36.75 103.255) (end 36.75 123) (width 4) (layer B.Cu) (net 11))
 (segment (start 41.25 127.5) (end 46 127.5) (width 4) (layer B.Cu) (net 11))
 (segment (start 46 104) (end 37.495 104) (width 4) (layer B.Cu) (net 11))
 (segment (start 37.495 104) (end 36.75 103.255) (width 4) (layer B.Cu) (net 11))
 (segment (start 36.75 96.245) (end 31.75 96.245) (width 4) (layer B.Cu) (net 11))
 (segment (start 36.75 103.255) (end 36.75 96.245) (width 4) (layer B.Cu) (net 11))
 (segment (start 31.75 103.255) (end 36.75 103.255) (width 4) (layer B.Cu) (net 11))
 (segment (start 55 104) (end 64 104) (width 4) (layer B.Cu) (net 9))
 (segment (start 64 119) (end 73 119) (width 4) (layer B.Cu) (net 8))
 (segment (start 73 104) (end 82 104) (width 4) (layer B.Cu) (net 7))
 (segment (start 82 119) (end 91 119) (width 4) (layer B.Cu) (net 6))
 (segment (start 91 104) (end 100 104) (width 4) (layer B.Cu) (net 5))
 (segment (start 100 119) (end 109 119) (width 4) (layer B.Cu) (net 4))
 (segment (start 109 104) (end 118 104) (width 4) (layer B.Cu) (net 3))
 (segment (start 118 119) (end 127 119) (width 4) (layer B.Cu) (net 2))
 (segment (start 127 127.5) (end 133.25 127.5) (width 4) (layer B.Cu) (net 1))
 (segment (start 136.25 124.5) (end 133.25 127.5) (width 4) (layer B.Cu) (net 1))
 (segment (start 136.25 103.255) (end 136.25 124.5) (width 4) (layer B.Cu) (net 1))
 (segment (start 135.505 104) (end 136.25 103.255) (width 4) (layer B.Cu) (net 1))
 (segment (start 127 104) (end 135.505 104) (width 4) (layer B.Cu) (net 1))
 (segment (start 127 57) (end 127 59) (width 4) (layer B.Cu) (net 1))
 (segment (start 127 59) (end 136.25 68.25) (width 4) (layer B.Cu) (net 1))
 (segment (start 135.5 80.5) (end 136.25 79.75) (width 4) (layer B.Cu) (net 1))
 (segment (start 127 80.5) (end 135.5 80.5) (width 4) (layer B.Cu) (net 1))
 (segment (start 136.25 68.25) (end 136.25 79.75) (width 4) (layer B.Cu) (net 1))
 (segment (start 136.25 79.75) (end 136.25 96.245) (width 4) (layer B.Cu) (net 1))
 (segment (start 136.25 96.245) (end 136.25 103.255) (width 4) (layer B.Cu) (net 1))
 (segment (start 141.25 96.245) (end 136.25 96.245) (width 4) (layer B.Cu) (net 1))
 (segment (start 141.25 103.255) (end 136.25 103.255) (width 4) (layer B.Cu) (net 1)))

